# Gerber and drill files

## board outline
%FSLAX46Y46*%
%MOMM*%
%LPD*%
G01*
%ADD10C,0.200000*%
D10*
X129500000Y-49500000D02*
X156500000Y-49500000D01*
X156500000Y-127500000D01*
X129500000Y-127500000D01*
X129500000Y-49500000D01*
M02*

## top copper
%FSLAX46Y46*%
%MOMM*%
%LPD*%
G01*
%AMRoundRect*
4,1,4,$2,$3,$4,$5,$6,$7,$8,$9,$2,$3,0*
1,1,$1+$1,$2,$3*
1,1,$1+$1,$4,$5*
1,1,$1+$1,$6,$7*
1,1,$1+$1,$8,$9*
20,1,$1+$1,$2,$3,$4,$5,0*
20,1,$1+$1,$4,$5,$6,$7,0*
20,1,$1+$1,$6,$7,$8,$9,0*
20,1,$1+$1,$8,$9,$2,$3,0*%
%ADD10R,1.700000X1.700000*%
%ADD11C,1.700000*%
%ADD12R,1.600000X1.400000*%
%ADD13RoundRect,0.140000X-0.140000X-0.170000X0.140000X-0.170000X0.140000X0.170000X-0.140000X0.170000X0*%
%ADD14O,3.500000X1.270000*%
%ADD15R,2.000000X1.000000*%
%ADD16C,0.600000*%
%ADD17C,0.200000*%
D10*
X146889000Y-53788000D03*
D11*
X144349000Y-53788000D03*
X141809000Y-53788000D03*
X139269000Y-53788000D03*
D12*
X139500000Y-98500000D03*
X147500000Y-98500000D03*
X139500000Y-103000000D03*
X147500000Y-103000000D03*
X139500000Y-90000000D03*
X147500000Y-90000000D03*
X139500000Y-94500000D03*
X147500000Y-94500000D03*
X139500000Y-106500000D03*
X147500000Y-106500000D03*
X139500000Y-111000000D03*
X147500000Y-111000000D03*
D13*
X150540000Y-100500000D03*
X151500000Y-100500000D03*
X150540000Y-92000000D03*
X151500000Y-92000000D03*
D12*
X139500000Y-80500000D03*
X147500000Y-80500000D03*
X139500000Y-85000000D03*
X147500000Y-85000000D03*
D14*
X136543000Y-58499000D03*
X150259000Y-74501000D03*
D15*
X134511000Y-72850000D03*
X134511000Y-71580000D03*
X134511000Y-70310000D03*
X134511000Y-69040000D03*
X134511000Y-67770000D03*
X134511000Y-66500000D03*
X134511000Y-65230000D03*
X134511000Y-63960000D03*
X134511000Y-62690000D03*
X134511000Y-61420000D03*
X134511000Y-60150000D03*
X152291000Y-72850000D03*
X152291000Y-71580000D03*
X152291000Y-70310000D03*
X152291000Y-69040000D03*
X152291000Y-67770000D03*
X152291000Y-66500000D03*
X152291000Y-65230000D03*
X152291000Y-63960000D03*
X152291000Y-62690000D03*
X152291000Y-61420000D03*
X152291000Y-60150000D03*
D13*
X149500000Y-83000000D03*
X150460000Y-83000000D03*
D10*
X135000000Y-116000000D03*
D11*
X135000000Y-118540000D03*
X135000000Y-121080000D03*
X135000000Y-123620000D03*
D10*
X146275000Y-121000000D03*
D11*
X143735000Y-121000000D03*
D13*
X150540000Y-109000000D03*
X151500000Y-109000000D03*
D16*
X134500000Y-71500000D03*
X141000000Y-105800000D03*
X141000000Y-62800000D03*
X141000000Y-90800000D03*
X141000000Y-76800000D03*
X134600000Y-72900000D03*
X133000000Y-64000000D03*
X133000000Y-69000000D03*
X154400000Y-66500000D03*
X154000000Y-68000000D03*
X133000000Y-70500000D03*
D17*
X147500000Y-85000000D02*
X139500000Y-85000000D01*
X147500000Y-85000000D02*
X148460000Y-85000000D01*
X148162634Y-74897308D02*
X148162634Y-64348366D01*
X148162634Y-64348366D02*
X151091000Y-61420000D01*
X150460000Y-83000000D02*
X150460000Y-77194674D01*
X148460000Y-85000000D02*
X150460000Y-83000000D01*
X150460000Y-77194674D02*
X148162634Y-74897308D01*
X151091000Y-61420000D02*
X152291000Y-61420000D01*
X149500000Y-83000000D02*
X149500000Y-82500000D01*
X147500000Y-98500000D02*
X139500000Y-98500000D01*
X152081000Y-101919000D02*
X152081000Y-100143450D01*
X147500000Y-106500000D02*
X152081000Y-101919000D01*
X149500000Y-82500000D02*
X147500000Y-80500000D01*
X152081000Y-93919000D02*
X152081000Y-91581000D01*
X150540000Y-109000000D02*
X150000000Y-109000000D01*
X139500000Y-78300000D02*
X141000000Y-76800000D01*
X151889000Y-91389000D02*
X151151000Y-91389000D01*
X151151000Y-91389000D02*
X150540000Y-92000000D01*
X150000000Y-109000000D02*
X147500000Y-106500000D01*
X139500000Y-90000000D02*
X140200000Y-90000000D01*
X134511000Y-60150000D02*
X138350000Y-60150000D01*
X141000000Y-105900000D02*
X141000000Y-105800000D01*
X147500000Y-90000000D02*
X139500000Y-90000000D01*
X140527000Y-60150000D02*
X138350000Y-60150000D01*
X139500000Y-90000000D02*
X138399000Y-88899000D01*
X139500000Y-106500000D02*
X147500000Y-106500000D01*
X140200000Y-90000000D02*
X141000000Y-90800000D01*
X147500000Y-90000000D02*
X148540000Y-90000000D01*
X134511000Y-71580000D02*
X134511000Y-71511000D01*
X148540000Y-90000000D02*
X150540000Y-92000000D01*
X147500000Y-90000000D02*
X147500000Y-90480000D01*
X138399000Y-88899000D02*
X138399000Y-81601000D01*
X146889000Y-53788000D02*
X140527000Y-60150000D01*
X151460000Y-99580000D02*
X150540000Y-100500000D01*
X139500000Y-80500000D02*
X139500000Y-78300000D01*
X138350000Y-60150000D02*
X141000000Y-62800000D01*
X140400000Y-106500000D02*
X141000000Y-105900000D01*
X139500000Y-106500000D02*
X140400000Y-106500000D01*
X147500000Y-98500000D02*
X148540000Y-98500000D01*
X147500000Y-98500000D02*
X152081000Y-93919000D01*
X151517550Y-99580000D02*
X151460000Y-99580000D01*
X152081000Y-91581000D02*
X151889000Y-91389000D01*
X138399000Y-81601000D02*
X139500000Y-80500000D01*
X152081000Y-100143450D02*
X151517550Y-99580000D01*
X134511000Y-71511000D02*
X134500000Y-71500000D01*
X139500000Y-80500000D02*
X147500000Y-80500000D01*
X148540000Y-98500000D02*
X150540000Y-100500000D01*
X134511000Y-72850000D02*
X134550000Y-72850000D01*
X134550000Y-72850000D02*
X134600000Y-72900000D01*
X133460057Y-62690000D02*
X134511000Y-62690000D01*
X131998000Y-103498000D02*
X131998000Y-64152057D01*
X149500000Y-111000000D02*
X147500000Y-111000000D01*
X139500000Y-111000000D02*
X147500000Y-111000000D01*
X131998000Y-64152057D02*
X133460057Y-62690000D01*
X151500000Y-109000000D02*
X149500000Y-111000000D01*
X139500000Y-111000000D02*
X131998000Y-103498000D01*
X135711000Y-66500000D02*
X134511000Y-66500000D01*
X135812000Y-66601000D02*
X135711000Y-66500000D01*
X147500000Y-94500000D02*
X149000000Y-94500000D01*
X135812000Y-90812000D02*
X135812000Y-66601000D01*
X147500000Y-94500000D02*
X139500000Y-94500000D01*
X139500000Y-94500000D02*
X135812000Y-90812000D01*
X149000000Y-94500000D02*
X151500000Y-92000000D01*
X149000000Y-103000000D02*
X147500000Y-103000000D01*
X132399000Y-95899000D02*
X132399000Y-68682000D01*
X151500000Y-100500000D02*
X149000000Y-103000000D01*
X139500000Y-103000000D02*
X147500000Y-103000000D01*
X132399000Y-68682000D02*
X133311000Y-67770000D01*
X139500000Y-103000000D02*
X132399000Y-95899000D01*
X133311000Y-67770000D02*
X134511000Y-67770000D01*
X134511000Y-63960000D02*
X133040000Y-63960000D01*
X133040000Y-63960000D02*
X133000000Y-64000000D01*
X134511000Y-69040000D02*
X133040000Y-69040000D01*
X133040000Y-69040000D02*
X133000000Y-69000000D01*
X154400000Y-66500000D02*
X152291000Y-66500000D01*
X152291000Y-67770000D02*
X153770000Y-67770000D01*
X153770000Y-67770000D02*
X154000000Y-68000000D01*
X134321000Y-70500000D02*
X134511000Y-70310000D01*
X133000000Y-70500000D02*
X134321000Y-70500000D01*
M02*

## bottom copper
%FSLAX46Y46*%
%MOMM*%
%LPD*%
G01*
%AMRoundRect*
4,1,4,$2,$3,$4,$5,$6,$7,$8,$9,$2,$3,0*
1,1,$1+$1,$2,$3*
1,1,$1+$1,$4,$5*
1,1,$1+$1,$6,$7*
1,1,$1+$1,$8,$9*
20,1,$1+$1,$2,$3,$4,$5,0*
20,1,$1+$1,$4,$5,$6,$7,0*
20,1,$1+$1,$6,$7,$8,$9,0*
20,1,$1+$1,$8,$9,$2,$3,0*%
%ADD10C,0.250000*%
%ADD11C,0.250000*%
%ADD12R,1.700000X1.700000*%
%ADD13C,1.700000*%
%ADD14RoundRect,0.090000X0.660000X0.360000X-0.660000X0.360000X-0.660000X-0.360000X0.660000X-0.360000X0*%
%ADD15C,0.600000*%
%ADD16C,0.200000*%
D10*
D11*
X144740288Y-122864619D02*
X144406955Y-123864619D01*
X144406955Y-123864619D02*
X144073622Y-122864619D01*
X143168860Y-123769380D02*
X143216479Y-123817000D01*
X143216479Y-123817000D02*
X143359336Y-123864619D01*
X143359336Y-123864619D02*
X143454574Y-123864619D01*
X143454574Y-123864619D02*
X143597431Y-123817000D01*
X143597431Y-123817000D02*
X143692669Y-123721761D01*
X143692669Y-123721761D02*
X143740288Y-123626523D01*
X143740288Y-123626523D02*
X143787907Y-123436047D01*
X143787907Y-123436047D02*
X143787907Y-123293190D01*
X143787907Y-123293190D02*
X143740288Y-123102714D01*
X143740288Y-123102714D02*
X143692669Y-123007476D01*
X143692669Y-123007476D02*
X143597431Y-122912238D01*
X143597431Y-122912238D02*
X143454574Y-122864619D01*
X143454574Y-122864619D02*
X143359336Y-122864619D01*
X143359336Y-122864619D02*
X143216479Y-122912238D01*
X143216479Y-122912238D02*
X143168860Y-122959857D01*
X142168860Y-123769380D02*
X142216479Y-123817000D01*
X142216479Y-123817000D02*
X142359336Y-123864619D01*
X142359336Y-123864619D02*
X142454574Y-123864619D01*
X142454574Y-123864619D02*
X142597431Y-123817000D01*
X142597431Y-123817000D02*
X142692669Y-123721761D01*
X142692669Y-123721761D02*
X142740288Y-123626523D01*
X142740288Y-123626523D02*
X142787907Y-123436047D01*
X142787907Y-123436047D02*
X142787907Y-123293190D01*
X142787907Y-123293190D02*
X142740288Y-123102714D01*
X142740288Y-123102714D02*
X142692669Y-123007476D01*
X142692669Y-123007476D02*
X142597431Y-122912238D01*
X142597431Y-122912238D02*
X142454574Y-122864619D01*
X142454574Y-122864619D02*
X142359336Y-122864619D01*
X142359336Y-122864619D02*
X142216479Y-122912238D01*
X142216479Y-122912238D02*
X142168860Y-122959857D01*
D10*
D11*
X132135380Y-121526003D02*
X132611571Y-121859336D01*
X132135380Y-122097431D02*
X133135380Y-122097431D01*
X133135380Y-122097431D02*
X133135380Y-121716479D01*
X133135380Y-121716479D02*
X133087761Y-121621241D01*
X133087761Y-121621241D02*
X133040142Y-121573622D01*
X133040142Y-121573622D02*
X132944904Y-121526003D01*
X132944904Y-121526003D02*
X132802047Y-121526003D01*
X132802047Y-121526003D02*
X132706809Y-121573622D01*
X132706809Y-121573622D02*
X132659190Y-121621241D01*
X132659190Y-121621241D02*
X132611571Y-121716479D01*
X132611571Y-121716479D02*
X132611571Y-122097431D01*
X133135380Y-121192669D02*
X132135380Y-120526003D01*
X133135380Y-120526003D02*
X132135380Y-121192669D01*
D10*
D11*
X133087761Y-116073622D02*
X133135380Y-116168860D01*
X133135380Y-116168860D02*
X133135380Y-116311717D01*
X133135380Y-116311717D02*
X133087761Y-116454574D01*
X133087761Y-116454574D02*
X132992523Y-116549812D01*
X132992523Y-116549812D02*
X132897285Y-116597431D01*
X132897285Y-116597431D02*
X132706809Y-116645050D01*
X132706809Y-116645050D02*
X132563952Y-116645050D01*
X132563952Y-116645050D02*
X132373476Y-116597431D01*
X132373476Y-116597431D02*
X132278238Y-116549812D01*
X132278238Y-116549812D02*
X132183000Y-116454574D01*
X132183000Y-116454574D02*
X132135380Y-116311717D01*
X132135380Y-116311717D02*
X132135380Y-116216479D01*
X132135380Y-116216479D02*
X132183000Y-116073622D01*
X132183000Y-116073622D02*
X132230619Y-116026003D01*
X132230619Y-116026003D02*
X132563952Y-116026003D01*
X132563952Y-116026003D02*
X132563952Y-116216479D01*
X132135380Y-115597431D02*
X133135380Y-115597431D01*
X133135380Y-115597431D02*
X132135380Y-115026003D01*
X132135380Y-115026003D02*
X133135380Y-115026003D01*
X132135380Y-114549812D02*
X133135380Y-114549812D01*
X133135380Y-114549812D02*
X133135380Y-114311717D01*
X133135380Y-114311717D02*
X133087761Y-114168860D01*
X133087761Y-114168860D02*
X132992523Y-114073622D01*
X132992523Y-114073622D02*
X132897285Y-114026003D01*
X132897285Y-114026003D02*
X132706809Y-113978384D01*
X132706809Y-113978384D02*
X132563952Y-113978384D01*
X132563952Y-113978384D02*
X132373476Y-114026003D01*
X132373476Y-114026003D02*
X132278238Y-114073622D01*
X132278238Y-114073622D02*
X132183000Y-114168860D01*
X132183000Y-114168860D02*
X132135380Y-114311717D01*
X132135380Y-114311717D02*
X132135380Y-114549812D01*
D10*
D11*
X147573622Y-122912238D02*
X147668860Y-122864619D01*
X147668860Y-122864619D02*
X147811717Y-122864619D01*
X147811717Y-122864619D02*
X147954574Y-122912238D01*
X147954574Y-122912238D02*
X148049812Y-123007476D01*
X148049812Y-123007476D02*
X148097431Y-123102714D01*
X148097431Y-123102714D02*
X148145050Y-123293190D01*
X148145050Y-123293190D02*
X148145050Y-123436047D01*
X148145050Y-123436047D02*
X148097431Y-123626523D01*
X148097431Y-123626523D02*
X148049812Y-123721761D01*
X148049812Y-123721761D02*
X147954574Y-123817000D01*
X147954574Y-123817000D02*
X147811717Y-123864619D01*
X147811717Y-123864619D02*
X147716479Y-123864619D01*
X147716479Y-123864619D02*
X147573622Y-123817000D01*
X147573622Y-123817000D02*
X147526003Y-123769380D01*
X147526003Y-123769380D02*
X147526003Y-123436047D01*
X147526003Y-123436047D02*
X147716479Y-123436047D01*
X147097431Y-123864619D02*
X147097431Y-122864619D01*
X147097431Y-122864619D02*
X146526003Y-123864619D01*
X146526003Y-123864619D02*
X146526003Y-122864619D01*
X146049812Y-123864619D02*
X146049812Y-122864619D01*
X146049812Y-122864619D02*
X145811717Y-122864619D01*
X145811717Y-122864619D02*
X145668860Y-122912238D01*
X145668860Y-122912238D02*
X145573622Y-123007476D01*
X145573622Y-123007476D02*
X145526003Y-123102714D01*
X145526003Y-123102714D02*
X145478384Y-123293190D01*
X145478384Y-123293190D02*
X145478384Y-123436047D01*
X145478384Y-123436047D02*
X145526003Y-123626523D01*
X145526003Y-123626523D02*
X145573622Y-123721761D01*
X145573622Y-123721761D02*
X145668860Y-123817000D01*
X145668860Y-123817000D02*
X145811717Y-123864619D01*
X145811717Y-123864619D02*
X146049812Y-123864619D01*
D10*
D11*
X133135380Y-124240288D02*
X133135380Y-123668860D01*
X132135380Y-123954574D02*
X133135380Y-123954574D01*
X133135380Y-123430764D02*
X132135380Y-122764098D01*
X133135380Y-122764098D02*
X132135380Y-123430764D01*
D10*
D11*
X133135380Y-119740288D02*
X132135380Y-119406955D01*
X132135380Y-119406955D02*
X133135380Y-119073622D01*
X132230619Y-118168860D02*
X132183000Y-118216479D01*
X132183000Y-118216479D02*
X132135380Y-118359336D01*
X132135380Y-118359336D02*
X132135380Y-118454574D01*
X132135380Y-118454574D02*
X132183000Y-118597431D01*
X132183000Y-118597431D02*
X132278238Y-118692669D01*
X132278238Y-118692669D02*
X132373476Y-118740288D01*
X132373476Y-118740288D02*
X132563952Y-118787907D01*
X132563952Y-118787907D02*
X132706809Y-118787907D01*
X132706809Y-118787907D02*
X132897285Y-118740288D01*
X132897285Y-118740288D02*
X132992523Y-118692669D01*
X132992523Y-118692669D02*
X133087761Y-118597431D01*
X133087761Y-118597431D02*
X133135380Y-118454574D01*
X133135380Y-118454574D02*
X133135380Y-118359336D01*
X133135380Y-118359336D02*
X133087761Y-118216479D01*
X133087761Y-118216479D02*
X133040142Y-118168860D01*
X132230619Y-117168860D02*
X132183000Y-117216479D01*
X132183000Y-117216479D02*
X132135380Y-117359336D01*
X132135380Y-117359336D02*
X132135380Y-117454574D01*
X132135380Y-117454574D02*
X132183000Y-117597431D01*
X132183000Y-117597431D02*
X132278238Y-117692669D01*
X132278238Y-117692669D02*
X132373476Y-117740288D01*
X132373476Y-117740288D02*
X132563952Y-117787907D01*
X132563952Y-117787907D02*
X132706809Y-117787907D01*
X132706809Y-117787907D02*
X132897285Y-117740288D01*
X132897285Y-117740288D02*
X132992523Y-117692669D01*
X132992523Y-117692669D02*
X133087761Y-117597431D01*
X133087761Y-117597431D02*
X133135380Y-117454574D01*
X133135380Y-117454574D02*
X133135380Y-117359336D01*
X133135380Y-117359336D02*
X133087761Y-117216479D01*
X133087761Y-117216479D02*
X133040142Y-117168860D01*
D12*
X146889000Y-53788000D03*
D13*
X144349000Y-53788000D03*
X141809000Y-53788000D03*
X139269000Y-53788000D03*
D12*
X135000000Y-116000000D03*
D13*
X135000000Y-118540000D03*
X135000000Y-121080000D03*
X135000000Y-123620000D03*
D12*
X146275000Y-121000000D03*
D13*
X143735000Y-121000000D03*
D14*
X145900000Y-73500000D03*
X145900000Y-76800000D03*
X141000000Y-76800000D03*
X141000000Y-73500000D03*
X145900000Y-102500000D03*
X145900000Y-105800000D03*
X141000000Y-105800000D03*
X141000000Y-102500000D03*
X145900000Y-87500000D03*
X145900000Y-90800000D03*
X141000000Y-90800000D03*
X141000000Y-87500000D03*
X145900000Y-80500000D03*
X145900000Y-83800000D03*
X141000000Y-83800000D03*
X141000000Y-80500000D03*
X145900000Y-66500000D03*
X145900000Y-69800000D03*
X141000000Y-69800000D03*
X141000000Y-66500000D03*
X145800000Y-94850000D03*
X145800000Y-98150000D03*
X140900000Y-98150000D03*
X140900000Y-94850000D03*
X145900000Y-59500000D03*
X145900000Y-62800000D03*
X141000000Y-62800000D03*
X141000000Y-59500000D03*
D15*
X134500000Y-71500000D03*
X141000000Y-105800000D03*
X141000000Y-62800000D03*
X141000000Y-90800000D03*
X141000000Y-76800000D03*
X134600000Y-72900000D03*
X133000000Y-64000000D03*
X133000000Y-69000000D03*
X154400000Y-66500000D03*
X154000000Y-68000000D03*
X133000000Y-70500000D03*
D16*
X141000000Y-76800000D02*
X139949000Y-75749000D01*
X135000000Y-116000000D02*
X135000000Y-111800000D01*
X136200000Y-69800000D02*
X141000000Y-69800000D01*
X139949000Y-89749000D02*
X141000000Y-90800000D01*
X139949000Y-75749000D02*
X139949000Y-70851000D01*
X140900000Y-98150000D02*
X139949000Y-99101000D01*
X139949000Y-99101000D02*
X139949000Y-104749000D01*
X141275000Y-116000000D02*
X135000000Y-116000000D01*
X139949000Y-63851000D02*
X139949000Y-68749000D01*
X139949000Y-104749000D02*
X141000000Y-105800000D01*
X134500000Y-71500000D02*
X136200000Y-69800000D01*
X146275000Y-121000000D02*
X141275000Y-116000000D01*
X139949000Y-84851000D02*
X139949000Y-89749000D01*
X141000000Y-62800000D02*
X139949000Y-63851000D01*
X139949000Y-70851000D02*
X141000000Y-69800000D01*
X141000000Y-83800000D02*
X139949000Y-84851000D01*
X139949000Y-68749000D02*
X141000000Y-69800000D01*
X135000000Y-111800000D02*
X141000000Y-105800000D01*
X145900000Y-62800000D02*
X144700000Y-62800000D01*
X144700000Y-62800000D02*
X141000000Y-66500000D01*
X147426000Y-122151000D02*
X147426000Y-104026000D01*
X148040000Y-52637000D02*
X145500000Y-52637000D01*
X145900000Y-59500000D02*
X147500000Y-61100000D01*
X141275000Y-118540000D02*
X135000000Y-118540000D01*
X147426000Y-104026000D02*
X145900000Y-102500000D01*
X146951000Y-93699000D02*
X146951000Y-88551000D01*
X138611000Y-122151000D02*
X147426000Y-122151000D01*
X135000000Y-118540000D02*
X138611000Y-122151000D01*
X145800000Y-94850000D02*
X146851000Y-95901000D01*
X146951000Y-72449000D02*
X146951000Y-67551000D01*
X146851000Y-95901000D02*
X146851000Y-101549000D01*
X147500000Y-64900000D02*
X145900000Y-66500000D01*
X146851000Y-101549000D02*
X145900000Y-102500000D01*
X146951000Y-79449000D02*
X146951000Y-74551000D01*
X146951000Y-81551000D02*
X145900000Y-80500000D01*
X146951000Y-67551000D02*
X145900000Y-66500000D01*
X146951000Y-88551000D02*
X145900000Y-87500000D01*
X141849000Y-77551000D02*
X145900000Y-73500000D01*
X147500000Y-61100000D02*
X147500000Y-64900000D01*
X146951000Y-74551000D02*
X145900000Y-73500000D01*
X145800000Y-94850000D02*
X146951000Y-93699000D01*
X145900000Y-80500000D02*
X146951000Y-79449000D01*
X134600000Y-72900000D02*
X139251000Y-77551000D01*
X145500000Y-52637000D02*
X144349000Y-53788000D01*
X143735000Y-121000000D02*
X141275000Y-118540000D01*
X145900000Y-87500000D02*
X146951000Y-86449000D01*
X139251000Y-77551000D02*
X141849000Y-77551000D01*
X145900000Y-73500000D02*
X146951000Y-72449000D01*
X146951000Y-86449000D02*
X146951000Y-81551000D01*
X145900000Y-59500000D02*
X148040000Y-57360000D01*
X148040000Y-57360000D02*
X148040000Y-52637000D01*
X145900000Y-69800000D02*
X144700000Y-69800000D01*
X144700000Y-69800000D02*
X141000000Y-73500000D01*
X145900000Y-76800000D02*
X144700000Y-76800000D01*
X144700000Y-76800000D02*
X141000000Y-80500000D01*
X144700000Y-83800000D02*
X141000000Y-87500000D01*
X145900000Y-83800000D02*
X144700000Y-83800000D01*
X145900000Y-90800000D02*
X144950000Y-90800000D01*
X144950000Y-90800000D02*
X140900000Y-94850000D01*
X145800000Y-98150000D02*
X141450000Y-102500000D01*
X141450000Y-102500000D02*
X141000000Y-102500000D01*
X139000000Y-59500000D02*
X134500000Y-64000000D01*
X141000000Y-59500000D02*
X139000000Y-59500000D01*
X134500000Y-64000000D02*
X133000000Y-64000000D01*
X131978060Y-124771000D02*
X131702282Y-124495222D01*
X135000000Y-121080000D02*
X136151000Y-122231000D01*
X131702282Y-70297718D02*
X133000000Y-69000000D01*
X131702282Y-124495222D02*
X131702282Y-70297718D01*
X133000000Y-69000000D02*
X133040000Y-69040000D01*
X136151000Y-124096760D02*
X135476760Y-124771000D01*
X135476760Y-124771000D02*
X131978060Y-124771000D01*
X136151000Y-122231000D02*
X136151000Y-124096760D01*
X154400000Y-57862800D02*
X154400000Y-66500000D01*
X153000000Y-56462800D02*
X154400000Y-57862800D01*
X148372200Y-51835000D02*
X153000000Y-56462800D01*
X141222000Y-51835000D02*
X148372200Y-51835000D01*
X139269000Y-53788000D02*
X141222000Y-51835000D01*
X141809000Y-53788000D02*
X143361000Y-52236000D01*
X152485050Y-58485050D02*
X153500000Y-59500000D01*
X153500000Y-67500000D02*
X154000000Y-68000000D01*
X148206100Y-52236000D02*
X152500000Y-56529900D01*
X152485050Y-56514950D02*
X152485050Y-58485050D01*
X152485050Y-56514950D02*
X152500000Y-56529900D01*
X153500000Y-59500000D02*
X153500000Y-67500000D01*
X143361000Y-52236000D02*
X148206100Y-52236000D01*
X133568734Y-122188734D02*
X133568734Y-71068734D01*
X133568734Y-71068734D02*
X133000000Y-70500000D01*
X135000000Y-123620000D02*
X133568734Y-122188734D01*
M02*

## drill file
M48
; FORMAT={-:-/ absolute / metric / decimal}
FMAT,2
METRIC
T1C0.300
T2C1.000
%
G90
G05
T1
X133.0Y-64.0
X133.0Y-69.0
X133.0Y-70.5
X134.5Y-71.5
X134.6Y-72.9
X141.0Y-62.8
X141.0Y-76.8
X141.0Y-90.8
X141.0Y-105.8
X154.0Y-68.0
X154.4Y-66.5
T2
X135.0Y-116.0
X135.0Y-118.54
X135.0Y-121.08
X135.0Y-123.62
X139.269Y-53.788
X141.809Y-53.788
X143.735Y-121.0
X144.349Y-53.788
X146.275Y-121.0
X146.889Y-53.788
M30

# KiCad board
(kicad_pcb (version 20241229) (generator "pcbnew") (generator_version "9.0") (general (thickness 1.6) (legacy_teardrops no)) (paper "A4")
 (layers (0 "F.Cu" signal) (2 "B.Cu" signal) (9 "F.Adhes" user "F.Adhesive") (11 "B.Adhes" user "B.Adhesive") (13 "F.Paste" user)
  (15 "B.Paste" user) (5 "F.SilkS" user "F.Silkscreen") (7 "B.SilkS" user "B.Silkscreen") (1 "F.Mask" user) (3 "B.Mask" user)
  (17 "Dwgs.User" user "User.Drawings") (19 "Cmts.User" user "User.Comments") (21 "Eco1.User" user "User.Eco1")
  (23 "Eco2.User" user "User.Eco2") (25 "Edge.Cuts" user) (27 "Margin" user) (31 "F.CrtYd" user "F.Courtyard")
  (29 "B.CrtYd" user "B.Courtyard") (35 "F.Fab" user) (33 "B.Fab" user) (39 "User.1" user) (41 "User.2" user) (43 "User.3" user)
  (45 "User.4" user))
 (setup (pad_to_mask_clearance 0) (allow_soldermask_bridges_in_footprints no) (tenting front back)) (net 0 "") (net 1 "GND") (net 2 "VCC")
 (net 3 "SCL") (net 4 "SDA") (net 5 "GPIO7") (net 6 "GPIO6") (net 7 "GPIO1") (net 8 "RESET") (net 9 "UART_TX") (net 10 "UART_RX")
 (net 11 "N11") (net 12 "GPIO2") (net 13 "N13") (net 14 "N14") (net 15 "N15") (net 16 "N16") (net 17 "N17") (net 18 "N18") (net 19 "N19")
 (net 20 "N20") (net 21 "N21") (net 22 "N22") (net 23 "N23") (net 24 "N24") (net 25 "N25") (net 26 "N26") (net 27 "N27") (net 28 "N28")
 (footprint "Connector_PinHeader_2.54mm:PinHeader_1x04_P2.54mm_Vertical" (layer "F.Cu") (at 146.889 53.788 -90)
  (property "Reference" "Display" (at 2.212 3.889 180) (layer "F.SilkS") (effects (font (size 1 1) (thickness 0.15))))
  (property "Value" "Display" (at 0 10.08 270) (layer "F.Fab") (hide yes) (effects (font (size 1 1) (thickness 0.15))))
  (pad "1" thru_hole rect (at 0 0 270) (size 1.7 1.7) (drill 1) (layers "*.Cu" "*.Mask") (remove_unused_layers no) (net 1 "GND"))
  (pad "2" thru_hole circle (at 0 2.54 270) (size 1.7 1.7) (drill 1) (layers "*.Cu" "*.Mask") (remove_unused_layers no) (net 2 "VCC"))
  (pad "3" thru_hole circle (at 0 5.08 270) (size 1.7 1.7) (drill 1) (layers "*.Cu" "*.Mask") (remove_unused_layers no) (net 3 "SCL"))
  (pad "4" thru_hole circle (at 0 7.62 270) (size 1.7 1.7) (drill 1) (layers "*.Cu" "*.Mask") (remove_unused_layers no) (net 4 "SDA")))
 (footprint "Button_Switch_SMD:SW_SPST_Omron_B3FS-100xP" (layer "F.Cu") (at 143.5 100.75)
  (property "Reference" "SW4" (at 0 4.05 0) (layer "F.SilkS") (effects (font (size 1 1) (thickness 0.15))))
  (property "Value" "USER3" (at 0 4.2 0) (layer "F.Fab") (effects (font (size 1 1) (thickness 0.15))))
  (pad "1" smd rect (at -4 -2.25 180) (size 1.6 1.4) (layers "F.Cu" "F.Mask" "F.Paste") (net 1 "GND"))
  (pad "1" smd rect (at 4 -2.25 180) (size 1.6 1.4) (layers "F.Cu" "F.Mask" "F.Paste") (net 1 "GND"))
  (pad "2" smd rect (at -4 2.25 180) (size 1.6 1.4) (layers "F.Cu" "F.Mask" "F.Paste") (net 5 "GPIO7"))
  (pad "2" smd rect (at 4 2.25 180) (size 1.6 1.4) (layers "F.Cu" "F.Mask" "F.Paste") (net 5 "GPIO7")))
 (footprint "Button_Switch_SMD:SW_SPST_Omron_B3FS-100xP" (layer "F.Cu") (at 143.5 92.25)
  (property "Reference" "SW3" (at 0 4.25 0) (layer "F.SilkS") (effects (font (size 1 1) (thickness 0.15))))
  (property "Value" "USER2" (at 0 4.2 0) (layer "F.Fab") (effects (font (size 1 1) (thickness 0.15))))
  (pad "1" smd rect (at -4 -2.25 180) (size 1.6 1.4) (layers "F.Cu" "F.Mask" "F.Paste") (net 1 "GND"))
  (pad "1" smd rect (at 4 -2.25 180) (size 1.6 1.4) (layers "F.Cu" "F.Mask" "F.Paste") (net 1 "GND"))
  (pad "2" smd rect (at -4 2.25 180) (size 1.6 1.4) (layers "F.Cu" "F.Mask" "F.Paste") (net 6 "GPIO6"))
  (pad "2" smd rect (at 4 2.25 180) (size 1.6 1.4) (layers "F.Cu" "F.Mask" "F.Paste") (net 6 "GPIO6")))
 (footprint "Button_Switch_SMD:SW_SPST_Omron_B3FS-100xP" (layer "F.Cu") (at 143.5 108.75)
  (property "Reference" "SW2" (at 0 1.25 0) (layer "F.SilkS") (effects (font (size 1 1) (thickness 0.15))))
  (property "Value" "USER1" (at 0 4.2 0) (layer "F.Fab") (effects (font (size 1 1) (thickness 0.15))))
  (pad "1" smd rect (at -4 -2.25 180) (size 1.6 1.4) (layers "F.Cu" "F.Mask" "F.Paste") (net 1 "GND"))
  (pad "1" smd rect (at 4 -2.25 180) (size 1.6 1.4) (layers "F.Cu" "F.Mask" "F.Paste") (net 1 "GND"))
  (pad "2" smd rect (at -4 2.25 180) (size 1.6 1.4) (layers "F.Cu" "F.Mask" "F.Paste") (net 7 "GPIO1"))
  (pad "2" smd rect (at 4 2.25 180) (size 1.6 1.4) (layers "F.Cu" "F.Mask" "F.Paste") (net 7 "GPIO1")))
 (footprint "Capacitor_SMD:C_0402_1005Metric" (layer "F.Cu") (at 151.02 100.5)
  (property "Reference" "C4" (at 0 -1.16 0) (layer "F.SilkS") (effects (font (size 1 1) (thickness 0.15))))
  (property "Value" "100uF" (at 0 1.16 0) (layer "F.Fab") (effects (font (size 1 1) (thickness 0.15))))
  (pad "1" smd roundrect (at -0.48 0) (size 0.56 0.62) (layers "F.Cu" "F.Mask" "F.Paste") (roundrect_rratio 0.25) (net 1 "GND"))
  (pad "2" smd roundrect (at 0.48 0) (size 0.56 0.62) (layers "F.Cu" "F.Mask" "F.Paste") (roundrect_rratio 0.25) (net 5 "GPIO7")))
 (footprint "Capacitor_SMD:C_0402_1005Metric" (layer "F.Cu") (at 151.02 92)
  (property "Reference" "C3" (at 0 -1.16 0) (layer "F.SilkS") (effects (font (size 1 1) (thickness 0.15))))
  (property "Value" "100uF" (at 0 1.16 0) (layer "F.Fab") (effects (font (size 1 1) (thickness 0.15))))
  (pad "1" smd roundrect (at -0.48 0) (size 0.56 0.62) (layers "F.Cu" "F.Mask" "F.Paste") (roundrect_rratio 0.25) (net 1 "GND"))
  (pad "2" smd roundrect (at 0.48 0) (size 0.56 0.62) (layers "F.Cu" "F.Mask" "F.Paste") (roundrect_rratio 0.25) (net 6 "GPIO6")))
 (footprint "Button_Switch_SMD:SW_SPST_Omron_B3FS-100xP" (layer "F.Cu") (at 143.5 82.75)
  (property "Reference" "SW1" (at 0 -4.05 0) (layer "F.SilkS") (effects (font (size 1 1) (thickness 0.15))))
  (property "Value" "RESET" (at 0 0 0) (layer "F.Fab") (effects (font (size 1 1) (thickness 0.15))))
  (pad "1" smd rect (at -4 -2.25 180) (size 1.6 1.4) (layers "F.Cu" "F.Mask" "F.Paste") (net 1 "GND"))
  (pad "1" smd rect (at 4 -2.25 180) (size 1.6 1.4) (layers "F.Cu" "F.Mask" "F.Paste") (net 1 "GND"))
  (pad "2" smd rect (at -4 2.25 180) (size 1.6 1.4) (layers "F.Cu" "F.Mask" "F.Paste") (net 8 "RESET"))
  (pad "2" smd rect (at 4 2.25 180) (size 1.6 1.4) (layers "F.Cu" "F.Mask" "F.Paste") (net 8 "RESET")))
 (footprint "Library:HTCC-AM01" (layer "F.Cu") (at 134.511 72.85)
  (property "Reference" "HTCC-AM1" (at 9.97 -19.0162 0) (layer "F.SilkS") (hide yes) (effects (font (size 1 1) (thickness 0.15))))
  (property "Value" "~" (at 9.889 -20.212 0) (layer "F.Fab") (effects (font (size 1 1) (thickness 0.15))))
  (pad "" smd oval (at 2.032 -14.351) (size 3.5 1.27) (layers "F.Cu" "F.Mask" "F.Paste"))
  (pad "" smd oval (at 15.748 1.651) (size 3.5 1.27) (layers "F.Cu" "F.Mask" "F.Paste"))
  (pad "1" smd rect (at 0 0 270) (size 1 2) (layers "F.Cu" "F.Mask" "F.Paste") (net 2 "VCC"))
  (pad "2" smd rect (at 0 -1.27 270) (size 1 2) (layers "F.Cu" "F.Mask" "F.Paste") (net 1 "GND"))
  (pad "3" smd rect (at 0 -2.54 90) (size 1 2) (layers "F.Cu" "F.Mask" "F.Paste") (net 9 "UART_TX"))
  (pad "4" smd rect (at 0 -3.81 90) (size 1 2) (layers "F.Cu" "F.Mask" "F.Paste") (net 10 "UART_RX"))
  (pad "5" smd rect (at 0 -5.08 90) (size 1 2) (layers "F.Cu" "F.Mask" "F.Paste") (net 5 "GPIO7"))
  (pad "6" smd rect (at 0 -6.35 90) (size 1 2) (layers "F.Cu" "F.Mask" "F.Paste") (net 6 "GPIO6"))
  (pad "7" smd rect (at 0 -7.62 90) (size 1 2) (layers "F.Cu" "F.Mask" "F.Paste") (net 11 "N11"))
  (pad "8" smd rect (at 0 -8.89 90) (size 1 2) (layers "F.Cu" "F.Mask" "F.Paste") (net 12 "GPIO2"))
  (pad "9" smd rect (at 0 -10.16 90) (size 1 2) (layers "F.Cu" "F.Mask" "F.Paste") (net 7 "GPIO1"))
  (pad "10" smd rect (at 0 -11.43 90) (size 1 2) (layers "F.Cu" "F.Mask" "F.Paste") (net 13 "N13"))
  (pad "11" smd rect (at 0 -12.7 90) (size 1 2) (layers "F.Cu" "F.Mask" "F.Paste") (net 1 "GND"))
  (pad "12" smd rect (at 17.78 0 270) (size 1 2) (layers "F.Cu" "F.Mask" "F.Paste") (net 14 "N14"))
  (pad "13" smd rect (at 17.78 -1.27 270) (size 1 2) (layers "F.Cu" "F.Mask" "F.Paste") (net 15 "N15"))
  (pad "14" smd rect (at 17.78 -2.54 90) (size 1 2) (layers "F.Cu" "F.Mask" "F.Paste") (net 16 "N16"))
  (pad "15" smd rect (at 17.78 -3.81 90) (size 1 2) (layers "F.Cu" "F.Mask" "F.Paste") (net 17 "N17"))
  (pad "16" smd rect (at 17.78 -5.08 90) (size 1 2) (layers "F.Cu" "F.Mask" "F.Paste") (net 3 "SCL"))
  (pad "17" smd rect (at 17.78 -6.35 90) (size 1 2) (layers "F.Cu" "F.Mask" "F.Paste") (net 4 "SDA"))
  (pad "18" smd rect (at 17.78 -7.62 90) (size 1 2) (layers "F.Cu" "F.Mask" "F.Paste") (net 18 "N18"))
  (pad "19" smd rect (at 17.78 -8.89 90) (size 1 2) (layers "F.Cu" "F.Mask" "F.Paste") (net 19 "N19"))
  (pad "20" smd rect (at 17.78 -10.16 90) (size 1 2) (layers "F.Cu" "F.Mask" "F.Paste") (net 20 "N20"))
  (pad "21" smd rect (at 17.78 -11.43 90) (size 1 2) (layers "F.Cu" "F.Mask" "F.Paste") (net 8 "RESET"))
  (pad "22" smd rect (at 17.78 -12.7 90) (size 1 2) (layers "F.Cu" "F.Mask" "F.Paste") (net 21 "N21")))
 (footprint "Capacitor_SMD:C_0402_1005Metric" (layer "F.Cu") (at 149.98 83)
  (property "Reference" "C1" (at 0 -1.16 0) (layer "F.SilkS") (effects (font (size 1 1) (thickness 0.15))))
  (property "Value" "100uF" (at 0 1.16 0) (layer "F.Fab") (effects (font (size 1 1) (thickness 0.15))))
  (pad "1" smd roundrect (at -0.48 0) (size 0.56 0.62) (layers "F.Cu" "F.Mask" "F.Paste") (roundrect_rratio 0.25) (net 1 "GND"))
  (pad "2" smd roundrect (at 0.48 0) (size 0.56 0.62) (layers "F.Cu" "F.Mask" "F.Paste") (roundrect_rratio 0.25) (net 8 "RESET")))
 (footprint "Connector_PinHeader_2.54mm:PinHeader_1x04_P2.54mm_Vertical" (layer "F.Cu") (at 135 116)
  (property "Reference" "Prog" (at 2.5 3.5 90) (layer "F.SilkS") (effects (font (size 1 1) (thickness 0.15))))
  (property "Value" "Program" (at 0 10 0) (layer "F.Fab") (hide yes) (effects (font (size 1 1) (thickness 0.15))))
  (pad "1" thru_hole rect (at 0 0) (size 1.7 1.7) (drill 1) (layers "*.Cu" "*.Mask") (remove_unused_layers no) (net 1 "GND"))
  (pad "2" thru_hole circle (at 0 2.54) (size 1.7 1.7) (drill 1) (layers "*.Cu" "*.Mask") (remove_unused_layers no) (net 2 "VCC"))
  (pad "3" thru_hole circle (at 0 5.08) (size 1.7 1.7) (drill 1) (layers "*.Cu" "*.Mask") (remove_unused_layers no) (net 10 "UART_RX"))
  (pad "4" thru_hole circle (at 0 7.62) (size 1.7 1.7) (drill 1) (layers "*.Cu" "*.Mask") (remove_unused_layers no) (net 9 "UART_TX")))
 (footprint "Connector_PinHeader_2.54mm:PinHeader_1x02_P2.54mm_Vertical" (layer "F.Cu") (at 146.275 121 -90)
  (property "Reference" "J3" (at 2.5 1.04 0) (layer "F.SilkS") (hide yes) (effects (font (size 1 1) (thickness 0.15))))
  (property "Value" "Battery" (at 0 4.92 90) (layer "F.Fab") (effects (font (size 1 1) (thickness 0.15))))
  (pad "1" thru_hole rect (at 0 0 270) (size 1.7 1.7) (drill 1) (layers "*.Cu" "*.Mask") (remove_unused_layers no) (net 1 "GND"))
  (pad "2" thru_hole circle (at 0 2.54 270) (size 1.7 1.7) (drill 1) (layers "*.Cu" "*.Mask") (remove_unused_layers no) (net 2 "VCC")))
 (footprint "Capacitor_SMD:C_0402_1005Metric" (layer "F.Cu") (at 151.02 109)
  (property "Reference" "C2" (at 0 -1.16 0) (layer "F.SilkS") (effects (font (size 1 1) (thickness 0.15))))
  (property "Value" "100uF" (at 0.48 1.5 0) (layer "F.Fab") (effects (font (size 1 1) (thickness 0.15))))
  (pad "1" smd roundrect (at -0.48 0) (size 0.56 0.62) (layers "F.Cu" "F.Mask" "F.Paste") (roundrect_rratio 0.25) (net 1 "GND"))
  (pad "2" smd roundrect (at 0.48 0) (size 0.56 0.62) (layers "F.Cu" "F.Mask" "F.Paste") (roundrect_rratio 0.25) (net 7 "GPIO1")))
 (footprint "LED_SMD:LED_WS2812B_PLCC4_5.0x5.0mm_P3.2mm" (layer "B.Cu") (at 143.45 75.15 180)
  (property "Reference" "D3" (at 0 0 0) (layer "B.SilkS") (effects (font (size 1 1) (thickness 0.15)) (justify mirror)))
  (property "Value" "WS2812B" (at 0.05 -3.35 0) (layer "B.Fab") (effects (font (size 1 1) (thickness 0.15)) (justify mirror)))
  (pad "1" smd roundrect (at -2.45 1.65 180) (size 1.5 0.9) (layers "B.Cu" "B.Mask" "B.Paste") (roundrect_rratio 0.1) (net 2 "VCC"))
  (pad "2" smd roundrect (at -2.45 -1.65 180) (size 1.5 0.9) (layers "B.Cu" "B.Mask" "B.Paste") (roundrect_rratio 0.1) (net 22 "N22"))
  (pad "3" smd roundrect (at 2.45 -1.65 180) (size 1.5 0.9) (layers "B.Cu" "B.Mask" "B.Paste") (roundrect_rratio 0.1) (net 1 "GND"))
  (pad "4" smd roundrect (at 2.45 1.65 180) (size 1.5 0.9) (layers "B.Cu" "B.Mask" "B.Paste") (roundrect_rratio 0.1) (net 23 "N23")))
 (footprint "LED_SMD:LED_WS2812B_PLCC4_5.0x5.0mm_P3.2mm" (layer "B.Cu") (at 143.45 104.15 180)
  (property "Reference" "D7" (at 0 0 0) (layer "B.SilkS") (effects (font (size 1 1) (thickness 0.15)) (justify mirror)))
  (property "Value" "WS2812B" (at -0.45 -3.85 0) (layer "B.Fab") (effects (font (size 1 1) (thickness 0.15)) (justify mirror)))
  (pad "1" smd roundrect (at -2.45 1.65 180) (size 1.5 0.9) (layers "B.Cu" "B.Mask" "B.Paste") (roundrect_rratio 0.1) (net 2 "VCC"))
  (pad "2" smd roundrect (at -2.45 -1.65 180) (size 1.5 0.9) (layers "B.Cu" "B.Mask" "B.Paste") (roundrect_rratio 0.1) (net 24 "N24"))
  (pad "3" smd roundrect (at 2.45 -1.65 180) (size 1.5 0.9) (layers "B.Cu" "B.Mask" "B.Paste") (roundrect_rratio 0.1) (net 1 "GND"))
  (pad "4" smd roundrect (at 2.45 1.65 180) (size 1.5 0.9) (layers "B.Cu" "B.Mask" "B.Paste") (roundrect_rratio 0.1) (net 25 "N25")))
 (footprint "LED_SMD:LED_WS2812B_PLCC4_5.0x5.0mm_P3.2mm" (layer "B.Cu") (at 143.45 89.15 180)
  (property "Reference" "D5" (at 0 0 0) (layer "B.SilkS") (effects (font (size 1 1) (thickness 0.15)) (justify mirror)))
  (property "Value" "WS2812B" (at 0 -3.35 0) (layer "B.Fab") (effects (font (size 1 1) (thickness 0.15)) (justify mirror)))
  (pad "1" smd roundrect (at -2.45 1.65 180) (size 1.5 0.9) (layers "B.Cu" "B.Mask" "B.Paste") (roundrect_rratio 0.1) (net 2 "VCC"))
  (pad "2" smd roundrect (at -2.45 -1.65 180) (size 1.5 0.9) (layers "B.Cu" "B.Mask" "B.Paste") (roundrect_rratio 0.1) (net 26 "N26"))
  (pad "3" smd roundrect (at 2.45 -1.65 180) (size 1.5 0.9) (layers "B.Cu" "B.Mask" "B.Paste") (roundrect_rratio 0.1) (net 1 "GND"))
  (pad "4" smd roundrect (at 2.45 1.65 180) (size 1.5 0.9) (layers "B.Cu" "B.Mask" "B.Paste") (roundrect_rratio 0.1) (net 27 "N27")))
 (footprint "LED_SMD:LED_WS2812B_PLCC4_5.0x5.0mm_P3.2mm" (layer "B.Cu") (at 143.45 82.15 180)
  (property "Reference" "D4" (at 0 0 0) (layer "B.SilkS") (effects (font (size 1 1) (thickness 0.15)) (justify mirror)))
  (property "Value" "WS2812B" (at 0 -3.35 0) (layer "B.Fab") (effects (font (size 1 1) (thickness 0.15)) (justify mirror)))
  (pad "1" smd roundrect (at -2.45 1.65 180) (size 1.5 0.9) (layers "B.Cu" "B.Mask" "B.Paste") (roundrect_rratio 0.1) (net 2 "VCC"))
  (pad "2" smd roundrect (at -2.45 -1.65 180) (size 1.5 0.9) (layers "B.Cu" "B.Mask" "B.Paste") (roundrect_rratio 0.1) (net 27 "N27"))
  (pad "3" smd roundrect (at 2.45 -1.65 180) (size 1.5 0.9) (layers "B.Cu" "B.Mask" "B.Paste") (roundrect_rratio 0.1) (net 1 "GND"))
  (pad "4" smd roundrect (at 2.45 1.65 180) (size 1.5 0.9) (layers "B.Cu" "B.Mask" "B.Paste") (roundrect_rratio 0.1) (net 22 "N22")))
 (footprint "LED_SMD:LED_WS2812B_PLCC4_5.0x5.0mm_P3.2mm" (layer "B.Cu") (at 143.45 68.15 180)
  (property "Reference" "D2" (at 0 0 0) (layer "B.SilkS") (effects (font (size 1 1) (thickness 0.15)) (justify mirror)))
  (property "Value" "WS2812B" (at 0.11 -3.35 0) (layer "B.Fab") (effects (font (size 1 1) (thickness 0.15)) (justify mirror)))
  (pad "1" smd roundrect (at -2.45 1.65 180) (size 1.5 0.9) (layers "B.Cu" "B.Mask" "B.Paste") (roundrect_rratio 0.1) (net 2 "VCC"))
  (pad "2" smd roundrect (at -2.45 -1.65 180) (size 1.5 0.9) (layers "B.Cu" "B.Mask" "B.Paste") (roundrect_rratio 0.1) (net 23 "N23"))
  (pad "3" smd roundrect (at 2.45 -1.65 180) (size 1.5 0.9) (layers "B.Cu" "B.Mask" "B.Paste") (roundrect_rratio 0.1) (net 1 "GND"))
  (pad "4" smd roundrect (at 2.45 1.65 180) (size 1.5 0.9) (layers "B.Cu" "B.Mask" "B.Paste") (roundrect_rratio 0.1) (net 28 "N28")))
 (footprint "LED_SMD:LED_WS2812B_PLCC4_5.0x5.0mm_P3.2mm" (layer "B.Cu") (at 143.35 96.5 180)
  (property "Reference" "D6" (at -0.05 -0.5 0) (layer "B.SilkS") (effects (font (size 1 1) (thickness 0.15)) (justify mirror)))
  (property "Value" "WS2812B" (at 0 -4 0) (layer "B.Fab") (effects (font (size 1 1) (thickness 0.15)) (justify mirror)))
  (pad "1" smd roundrect (at -2.45 1.65 180) (size 1.5 0.9) (layers "B.Cu" "B.Mask" "B.Paste") (roundrect_rratio 0.1) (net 2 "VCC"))
  (pad "2" smd roundrect (at -2.45 -1.65 180) (size 1.5 0.9) (layers "B.Cu" "B.Mask" "B.Paste") (roundrect_rratio 0.1) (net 25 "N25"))
  (pad "3" smd roundrect (at 2.45 -1.65 180) (size 1.5 0.9) (layers "B.Cu" "B.Mask" "B.Paste") (roundrect_rratio 0.1) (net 1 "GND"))
  (pad "4" smd roundrect (at 2.45 1.65 180) (size 1.5 0.9) (layers "B.Cu" "B.Mask" "B.Paste") (roundrect_rratio 0.1) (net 26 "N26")))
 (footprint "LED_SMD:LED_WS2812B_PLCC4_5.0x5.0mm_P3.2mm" (layer "B.Cu") (at 143.45 61.15 180)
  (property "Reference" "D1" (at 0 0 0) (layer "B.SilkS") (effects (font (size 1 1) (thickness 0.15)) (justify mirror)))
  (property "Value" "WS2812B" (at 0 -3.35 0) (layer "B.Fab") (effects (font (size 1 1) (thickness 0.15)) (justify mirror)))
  (pad "1" smd roundrect (at -2.45 1.65 180) (size 1.5 0.9) (layers "B.Cu" "B.Mask" "B.Paste") (roundrect_rratio 0.1) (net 2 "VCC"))
  (pad "2" smd roundrect (at -2.45 -1.65 180) (size 1.5 0.9) (layers "B.Cu" "B.Mask" "B.Paste") (roundrect_rratio 0.1) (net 28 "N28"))
  (pad "3" smd roundrect (at 2.45 -1.65 180) (size 1.5 0.9) (layers "B.Cu" "B.Mask" "B.Paste") (roundrect_rratio 0.1) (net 1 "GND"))
  (pad "4" smd roundrect (at 2.45 1.65 180) (size 1.5 0.9) (layers "B.Cu" "B.Mask" "B.Paste") (roundrect_rratio 0.1) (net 12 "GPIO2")))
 (gr_rect (start 129.5 49.5) (end 156.5 127.5) (stroke (width 0.2) (type solid)) (fill no) (layer "Edge.Cuts"))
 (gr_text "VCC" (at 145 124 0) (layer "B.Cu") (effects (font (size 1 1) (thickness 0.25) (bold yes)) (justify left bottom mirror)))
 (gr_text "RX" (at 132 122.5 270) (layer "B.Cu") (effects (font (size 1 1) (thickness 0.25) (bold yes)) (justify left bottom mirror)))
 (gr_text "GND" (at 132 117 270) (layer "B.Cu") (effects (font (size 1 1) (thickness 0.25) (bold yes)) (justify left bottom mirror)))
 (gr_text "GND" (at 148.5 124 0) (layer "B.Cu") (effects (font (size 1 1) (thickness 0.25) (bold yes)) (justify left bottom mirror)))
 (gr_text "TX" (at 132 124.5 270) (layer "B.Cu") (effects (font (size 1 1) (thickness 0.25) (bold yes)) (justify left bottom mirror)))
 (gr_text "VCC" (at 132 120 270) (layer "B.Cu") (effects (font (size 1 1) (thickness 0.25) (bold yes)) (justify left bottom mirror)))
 (segment (start 147.5 85) (end 139.5 85) (width 0.2) (layer "F.Cu") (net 8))
 (segment (start 147.5 85) (end 148.46 85) (width 0.2) (layer "F.Cu") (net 8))
 (segment (start 148.162634 74.897308) (end 148.162634 64.348366) (width 0.2) (layer "F.Cu") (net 8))
 (segment (start 148.162634 64.348366) (end 151.091 61.42) (width 0.2) (layer "F.Cu") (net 8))
 (segment (start 150.46 83) (end 150.46 77.194674) (width 0.2) (layer "F.Cu") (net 8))
 (segment (start 148.46 85) (end 150.46 83) (width 0.2) (layer "F.Cu") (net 8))
 (segment (start 150.46 77.194674) (end 148.162634 74.897308) (width 0.2) (layer "F.Cu") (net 8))
 (segment (start 151.091 61.42) (end 152.291 61.42) (width 0.2) (layer "F.Cu") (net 8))
 (segment (start 149.5 83) (end 149.5 82.5) (width 0.2) (layer "F.Cu") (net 1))
 (segment (start 147.5 98.5) (end 139.5 98.5) (width 0.2) (layer "F.Cu") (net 1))
 (segment (start 152.081 101.919) (end 152.081 100.14345) (width 0.2) (layer "F.Cu") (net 1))
 (segment (start 147.5 106.5) (end 152.081 101.919) (width 0.2) (layer "F.Cu") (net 1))
 (segment (start 149.5 82.5) (end 147.5 80.5) (width 0.2) (layer "F.Cu") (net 1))
 (segment (start 152.081 93.919) (end 152.081 91.581) (width 0.2) (layer "F.Cu") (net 1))
 (segment (start 150.54 109) (end 150 109) (width 0.2) (layer "F.Cu") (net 1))
 (segment (start 139.5 78.3) (end 141 76.8) (width 0.2) (layer "F.Cu") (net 1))
 (segment (start 151.889 91.389) (end 151.151 91.389) (width 0.2) (layer "F.Cu") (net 1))
 (segment (start 151.151 91.389) (end 150.54 92) (width 0.2) (layer "F.Cu") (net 1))
 (segment (start 150 109) (end 147.5 106.5) (width 0.2) (layer "F.Cu") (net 1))
 (segment (start 139.5 90) (end 140.2 90) (width 0.2) (layer "F.Cu") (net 1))
 (segment (start 134.511 60.15) (end 138.35 60.15) (width 0.2) (layer "F.Cu") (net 1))
 (segment (start 141 105.9) (end 141 105.8) (width 0.2) (layer "F.Cu") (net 1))
 (segment (start 147.5 90) (end 139.5 90) (width 0.2) (layer "F.Cu") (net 1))
 (segment (start 140.527 60.15) (end 138.35 60.15) (width 0.2) (layer "F.Cu") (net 1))
 (segment (start 139.5 90) (end 138.399 88.899) (width 0.2) (layer "F.Cu") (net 1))
 (segment (start 139.5 106.5) (end 147.5 106.5) (width 0.2) (layer "F.Cu") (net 1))
 (segment (start 140.2 90) (end 141 90.8) (width 0.2) (layer "F.Cu") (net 1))
 (segment (start 147.5 90) (end 148.54 90) (width 0.2) (layer "F.Cu") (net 1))
 (segment (start 134.511 71.58) (end 134.511 71.511) (width 0.2) (layer "F.Cu") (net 1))
 (segment (start 148.54 90) (end 150.54 92) (width 0.2) (layer "F.Cu") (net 1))
 (segment (start 147.5 90) (end 147.5 90.48) (width 0.2) (layer "F.Cu") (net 1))
 (segment (start 138.399 88.899) (end 138.399 81.601) (width 0.2) (layer "F.Cu") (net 1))
 (segment (start 146.889 53.788) (end 140.527 60.15) (width 0.2) (layer "F.Cu") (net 1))
 (segment (start 151.46 99.58) (end 150.54 100.5) (width 0.2) (layer "F.Cu") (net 1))
 (segment (start 139.5 80.5) (end 139.5 78.3) (width 0.2) (layer "F.Cu") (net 1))
 (segment (start 138.35 60.15) (end 141 62.8) (width 0.2) (layer "F.Cu") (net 1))
 (segment (start 140.4 106.5) (end 141 105.9) (width 0.2) (layer "F.Cu") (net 1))
 (segment (start 139.5 106.5) (end 140.4 106.5) (width 0.2) (layer "F.Cu") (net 1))
 (segment (start 147.5 98.5) (end 148.54 98.5) (width 0.2) (layer "F.Cu") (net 1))
 (segment (start 147.5 98.5) (end 152.081 93.919) (width 0.2) (layer "F.Cu") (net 1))
 (segment (start 151.51755 99.58) (end 151.46 99.58) (width 0.2) (layer "F.Cu") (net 1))
 (segment (start 152.081 91.581) (end 151.889 91.389) (width 0.2) (layer "F.Cu") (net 1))
 (segment (start 138.399 81.601) (end 139.5 80.5) (width 0.2) (layer "F.Cu") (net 1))
 (segment (start 152.081 100.14345) (end 151.51755 99.58) (width 0.2) (layer "F.Cu") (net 1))
 (segment (start 134.511 71.511) (end 134.5 71.5) (width 0.2) (layer "F.Cu") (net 1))
 (segment (start 139.5 80.5) (end 147.5 80.5) (width 0.2) (layer "F.Cu") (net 1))
 (segment (start 148.54 98.5) (end 150.54 100.5) (width 0.2) (layer "F.Cu") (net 1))
 (via (at 134.5 71.5) (size 0.6) (drill 0.3) (layers "F.Cu" "B.Cu") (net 1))
 (via (at 141 105.8) (size 0.6) (drill 0.3) (layers "F.Cu" "B.Cu") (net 1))
 (via (at 141 62.8) (size 0.6) (drill 0.3) (layers "F.Cu" "B.Cu") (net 1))
 (via (at 141 90.8) (size 0.6) (drill 0.3) (layers "F.Cu" "B.Cu") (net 1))
 (via (at 141 76.8) (size 0.6) (drill 0.3) (layers "F.Cu" "B.Cu") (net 1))
 (segment (start 141 76.8) (end 139.949 75.749) (width 0.2) (layer "B.Cu") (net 1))
 (segment (start 135 116) (end 135 111.8) (width 0.2) (layer "B.Cu") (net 1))
 (segment (start 136.2 69.8) (end 141 69.8) (width 0.2) (layer "B.Cu") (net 1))
 (segment (start 139.949 89.749) (end 141 90.8) (width 0.2) (layer "B.Cu") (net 1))
 (segment (start 139.949 75.749) (end 139.949 70.851) (width 0.2) (layer "B.Cu") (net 1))
 (segment (start 140.9 98.15) (end 139.949 99.101) (width 0.2) (layer "B.Cu") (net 1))
 (segment (start 139.949 99.101) (end 139.949 104.749) (width 0.2) (layer "B.Cu") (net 1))
 (segment (start 141.275 116) (end 135 116) (width 0.2) (layer "B.Cu") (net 1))
 (segment (start 139.949 63.851) (end 139.949 68.749) (width 0.2) (layer "B.Cu") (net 1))
 (segment (start 139.949 104.749) (end 141 105.8) (width 0.2) (layer "B.Cu") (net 1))
 (segment (start 134.5 71.5) (end 136.2 69.8) (width 0.2) (layer "B.Cu") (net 1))
 (segment (start 146.275 121) (end 141.275 116) (width 0.2) (layer "B.Cu") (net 1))
 (segment (start 139.949 84.851) (end 139.949 89.749) (width 0.2) (layer "B.Cu") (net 1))
 (segment (start 141 62.8) (end 139.949 63.851) (width 0.2) (layer "B.Cu") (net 1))
 (segment (start 139.949 70.851) (end 141 69.8) (width 0.2) (layer "B.Cu") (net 1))
 (segment (start 141 83.8) (end 139.949 84.851) (width 0.2) (layer "B.Cu") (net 1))
 (segment (start 139.949 68.749) (end 141 69.8) (width 0.2) (layer "B.Cu") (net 1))
 (segment (start 135 111.8) (end 141 105.8) (width 0.2) (layer "B.Cu") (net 1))
 (segment (start 145.9 62.8) (end 144.7 62.8) (width 0.2) (layer "B.Cu") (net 28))
 (segment (start 144.7 62.8) (end 141 66.5) (width 0.2) (layer "B.Cu") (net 28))
 (segment (start 134.511 72.85) (end 134.55 72.85) (width 0.2) (layer "F.Cu") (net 2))
 (segment (start 134.55 72.85) (end 134.6 72.9) (width 0.2) (layer "F.Cu") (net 2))
 (via (at 134.6 72.9) (size 0.6) (drill 0.3) (layers "F.Cu" "B.Cu") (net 2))
 (segment (start 147.426 122.151) (end 147.426 104.026) (width 0.2) (layer "B.Cu") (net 2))
 (segment (start 148.04 52.637) (end 145.5 52.637) (width 0.2) (layer "B.Cu") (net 2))
 (segment (start 145.9 59.5) (end 147.5 61.1) (width 0.2) (layer "B.Cu") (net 2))
 (segment (start 141.275 118.54) (end 135 118.54) (width 0.2) (layer "B.Cu") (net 2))
 (segment (start 147.426 104.026) (end 145.9 102.5) (width 0.2) (layer "B.Cu") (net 2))
 (segment (start 146.951 93.699) (end 146.951 88.551) (width 0.2) (layer "B.Cu") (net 2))
 (segment (start 138.611 122.151) (end 147.426 122.151) (width 0.2) (layer "B.Cu") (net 2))
 (segment (start 135 118.54) (end 138.611 122.151) (width 0.2) (layer "B.Cu") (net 2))
 (segment (start 145.8 94.85) (end 146.851 95.901) (width 0.2) (layer "B.Cu") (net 2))
 (segment (start 146.951 72.449) (end 146.951 67.551) (width 0.2) (layer "B.Cu") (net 2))
 (segment (start 146.851 95.901) (end 146.851 101.549) (width 0.2) (layer "B.Cu") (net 2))
 (segment (start 147.5 64.9) (end 145.9 66.5) (width 0.2) (layer "B.Cu") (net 2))
 (segment (start 146.851 101.549) (end 145.9 102.5) (width 0.2) (layer "B.Cu") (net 2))
 (segment (start 146.951 79.449) (end 146.951 74.551) (width 0.2) (layer "B.Cu") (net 2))
 (segment (start 146.951 81.551) (end 145.9 80.5) (width 0.2) (layer "B.Cu") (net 2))
 (segment (start 146.951 67.551) (end 145.9 66.5) (width 0.2) (layer "B.Cu") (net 2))
 (segment (start 146.951 88.551) (end 145.9 87.5) (width 0.2) (layer "B.Cu") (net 2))
 (segment (start 141.849 77.551) (end 145.9 73.5) (width 0.2) (layer "B.Cu") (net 2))
 (segment (start 147.5 61.1) (end 147.5 64.9) (width 0.2) (layer "B.Cu") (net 2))
 (segment (start 146.951 74.551) (end 145.9 73.5) (width 0.2) (layer "B.Cu") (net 2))
 (segment (start 145.8 94.85) (end 146.951 93.699) (width 0.2) (layer "B.Cu") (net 2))
 (segment (start 145.9 80.5) (end 146.951 79.449) (width 0.2) (layer "B.Cu") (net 2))
 (segment (start 134.6 72.9) (end 139.251 77.551) (width 0.2) (layer "B.Cu") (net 2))
 (segment (start 145.5 52.637) (end 144.349 53.788) (width 0.2) (layer "B.Cu") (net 2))
 (segment (start 143.735 121) (end 141.275 118.54) (width 0.2) (layer "B.Cu") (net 2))
 (segment (start 145.9 87.5) (end 146.951 86.449) (width 0.2) (layer "B.Cu") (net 2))
 (segment (start 139.251 77.551) (end 141.849 77.551) (width 0.2) (layer "B.Cu") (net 2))
 (segment (start 145.9 73.5) (end 146.951 72.449) (width 0.2) (layer "B.Cu") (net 2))
 (segment (start 146.951 86.449) (end 146.951 81.551) (width 0.2) (layer "B.Cu") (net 2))
 (segment (start 145.9 59.5) (end 148.04 57.36) (width 0.2) (layer "B.Cu") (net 2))
 (segment (start 148.04 57.36) (end 148.04 52.637) (width 0.2) (layer "B.Cu") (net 2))
 (segment (start 145.9 69.8) (end 144.7 69.8) (width 0.2) (layer "B.Cu") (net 23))
 (segment (start 144.7 69.8) (end 141 73.5) (width 0.2) (layer "B.Cu") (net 23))
 (segment (start 145.9 76.8) (end 144.7 76.8) (width 0.2) (layer "B.Cu") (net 22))
 (segment (start 144.7 76.8) (end 141 80.5) (width 0.2) (layer "B.Cu") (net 22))
 (segment (start 144.7 83.8) (end 141 87.5) (width 0.2) (layer "B.Cu") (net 27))
 (segment (start 145.9 83.8) (end 144.7 83.8) (width 0.2) (layer "B.Cu") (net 27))
 (segment (start 145.9 90.8) (end 144.95 90.8) (width 0.2) (layer "B.Cu") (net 26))
 (segment (start 144.95 90.8) (end 140.9 94.85) (width 0.2) (layer "B.Cu") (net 26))
 (segment (start 145.8 98.15) (end 141.45 102.5) (width 0.2) (layer "B.Cu") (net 25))
 (segment (start 141.45 102.5) (end 141 102.5) (width 0.2) (layer "B.Cu") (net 25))
 (segment (start 133.460057 62.69) (end 134.511 62.69) (width 0.2) (layer "F.Cu") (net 7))
 (segment (start 131.998 103.498) (end 131.998 64.152057) (width 0.2) (layer "F.Cu") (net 7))
 (segment (start 149.5 111) (end 147.5 111) (width 0.2) (layer "F.Cu") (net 7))
 (segment (start 139.5 111) (end 147.5 111) (width 0.2) (layer "F.Cu") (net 7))
 (segment (start 131.998 64.152057) (end 133.460057 62.69) (width 0.2) (layer "F.Cu") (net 7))
 (segment (start 151.5 109) (end 149.5 111) (width 0.2) (layer "F.Cu") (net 7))
 (segment (start 139.5 111) (end 131.998 103.498) (width 0.2) (layer "F.Cu") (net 7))
 (segment (start 135.711 66.5) (end 134.511 66.5) (width 0.2) (layer "F.Cu") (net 6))
 (segment (start 135.812 66.601) (end 135.711 66.5) (width 0.2) (layer "F.Cu") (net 6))
 (segment (start 147.5 94.5) (end 149 94.5) (width 0.2) (layer "F.Cu") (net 6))
 (segment (start 135.812 90.812) (end 135.812 66.601) (width 0.2) (layer "F.Cu") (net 6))
 (segment (start 147.5 94.5) (end 139.5 94.5) (width 0.2) (layer "F.Cu") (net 6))
 (segment (start 139.5 94.5) (end 135.812 90.812) (width 0.2) (layer "F.Cu") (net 6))
 (segment (start 149 94.5) (end 151.5 92) (width 0.2) (layer "F.Cu") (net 6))
 (segment (start 149 103) (end 147.5 103) (width 0.2) (layer "F.Cu") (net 5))
 (segment (start 132.399 95.899) (end 132.399 68.682) (width 0.2) (layer "F.Cu") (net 5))
 (segment (start 151.5 100.5) (end 149 103) (width 0.2) (layer "F.Cu") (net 5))
 (segment (start 139.5 103) (end 147.5 103) (width 0.2) (layer "F.Cu") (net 5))
 (segment (start 132.399 68.682) (end 133.311 67.77) (width 0.2) (layer "F.Cu") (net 5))
 (segment (start 139.5 103) (end 132.399 95.899) (width 0.2) (layer "F.Cu") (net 5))
 (segment (start 133.311 67.77) (end 134.511 67.77) (width 0.2) (layer "F.Cu") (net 5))
 (segment (start 134.511 63.96) (end 133.04 63.96) (width 0.2) (layer "F.Cu") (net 12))
 (segment (start 133.04 63.96) (end 133 64) (width 0.2) (layer "F.Cu") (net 12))
 (via (at 133 64) (size 0.6) (drill 0.3) (layers "F.Cu" "B.Cu") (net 12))
 (segment (start 139 59.5) (end 134.5 64) (width 0.2) (layer "B.Cu") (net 12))
 (segment (start 141 59.5) (end 139 59.5) (width 0.2) (layer "B.Cu") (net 12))
 (segment (start 134.5 64) (end 133 64) (width 0.2) (layer "B.Cu") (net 12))
 (segment (start 134.511 69.04) (end 133.04 69.04) (width 0.2) (layer "F.Cu") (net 10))
 (segment (start 133.04 69.04) (end 133 69) (width 0.2) (layer "F.Cu") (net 10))
 (via (at 133 69) (size 0.6) (drill 0.3) (layers "F.Cu" "B.Cu") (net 10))
 (segment (start 131.97806 124.771) (end 131.702282 124.495222) (width 0.2) (layer "B.Cu") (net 10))
 (segment (start 135 121.08) (end 136.151 122.231) (width 0.2) (layer "B.Cu") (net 10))
 (segment (start 131.702282 70.297718) (end 133 69) (width 0.2) (layer "B.Cu") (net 10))
 (segment (start 131.702282 124.495222) (end 131.702282 70.297718) (width 0.2) (layer "B.Cu") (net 10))
 (segment (start 133 69) (end 133.04 69.04) (width 0.2) (layer "B.Cu") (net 10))
 (segment (start 136.151 124.09676) (end 135.47676 124.771) (width 0.2) (layer "B.Cu") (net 10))
 (segment (start 135.47676 124.771) (end 131.97806 124.771) (width 0.2) (layer "B.Cu") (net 10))
 (segment (start 136.151 122.231) (end 136.151 124.09676) (width 0.2) (layer "B.Cu") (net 10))
 (segment (start 154.4 66.5) (end 152.291 66.5) (width 0.2) (layer "F.Cu") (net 4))
 (via (at 154.4 66.5) (size 0.6) (drill 0.3) (layers "F.Cu" "B.Cu") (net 4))
 (segment (start 154.4 57.8628) (end 154.4 66.5) (width 0.2) (layer "B.Cu") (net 4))
 (segment (start 153 56.4628) (end 154.4 57.8628) (width 0.2) (layer "B.Cu") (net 4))
 (segment (start 148.3722 51.835) (end 153 56.4628) (width 0.2) (layer "B.Cu") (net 4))
 (segment (start 141.222 51.835) (end 148.3722 51.835) (width 0.2) (layer "B.Cu") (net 4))
 (segment (start 139.269 53.788) (end 141.222 51.835) (width 0.2) (layer "B.Cu") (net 4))
 (segment (start 152.291 67.77) (end 153.77 67.77) (width 0.2) (layer "F.Cu") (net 3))
 (segment (start 153.77 67.77) (end 154 68) (width 0.2) (layer "F.Cu") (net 3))
 (via (at 154 68) (size 0.6) (drill 0.3) (layers "F.Cu" "B.Cu") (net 3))
 (segment (start 141.809 53.788) (end 143.361 52.236) (width 0.2) (layer "B.Cu") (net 3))
 (segment (start 152.48505 58.48505) (end 153.5 59.5) (width 0.2) (layer "B.Cu") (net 3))
 (segment (start 153.5 67.5) (end 154 68) (width 0.2) (layer "B.Cu") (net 3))
 (segment (start 148.2061 52.236) (end 152.5 56.5299) (width 0.2) (layer "B.Cu") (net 3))
 (segment (start 152.48505 56.51495) (end 152.48505 58.48505) (width 0.2) (layer "B.Cu") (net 3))
 (segment (start 152.48505 56.51495) (end 152.5 56.5299) (width 0.2) (layer "B.Cu") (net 3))
 (segment (start 153.5 59.5) (end 153.5 67.5) (width 0.2) (layer "B.Cu") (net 3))
 (segment (start 143.361 52.236) (end 148.2061 52.236) (width 0.2) (layer "B.Cu") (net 3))
 (segment (start 134.321 70.5) (end 134.511 70.31) (width 0.2) (layer "F.Cu") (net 9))
 (segment (start 133 70.5) (end 134.321 70.5) (width 0.2) (layer "F.Cu") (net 9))
 (via (at 133 70.5) (size 0.6) (drill 0.3) (layers "F.Cu" "B.Cu") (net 9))
 (segment (start 133.568734 122.188734) (end 133.568734 71.068734) (width 0.2) (layer "B.Cu") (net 9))
 (segment (start 133.568734 71.068734) (end 133 70.5) (width 0.2) (layer "B.Cu") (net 9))
 (segment (start 135 123.62) (end 133.568734 122.188734) (width 0.2) (layer "B.Cu") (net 9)))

